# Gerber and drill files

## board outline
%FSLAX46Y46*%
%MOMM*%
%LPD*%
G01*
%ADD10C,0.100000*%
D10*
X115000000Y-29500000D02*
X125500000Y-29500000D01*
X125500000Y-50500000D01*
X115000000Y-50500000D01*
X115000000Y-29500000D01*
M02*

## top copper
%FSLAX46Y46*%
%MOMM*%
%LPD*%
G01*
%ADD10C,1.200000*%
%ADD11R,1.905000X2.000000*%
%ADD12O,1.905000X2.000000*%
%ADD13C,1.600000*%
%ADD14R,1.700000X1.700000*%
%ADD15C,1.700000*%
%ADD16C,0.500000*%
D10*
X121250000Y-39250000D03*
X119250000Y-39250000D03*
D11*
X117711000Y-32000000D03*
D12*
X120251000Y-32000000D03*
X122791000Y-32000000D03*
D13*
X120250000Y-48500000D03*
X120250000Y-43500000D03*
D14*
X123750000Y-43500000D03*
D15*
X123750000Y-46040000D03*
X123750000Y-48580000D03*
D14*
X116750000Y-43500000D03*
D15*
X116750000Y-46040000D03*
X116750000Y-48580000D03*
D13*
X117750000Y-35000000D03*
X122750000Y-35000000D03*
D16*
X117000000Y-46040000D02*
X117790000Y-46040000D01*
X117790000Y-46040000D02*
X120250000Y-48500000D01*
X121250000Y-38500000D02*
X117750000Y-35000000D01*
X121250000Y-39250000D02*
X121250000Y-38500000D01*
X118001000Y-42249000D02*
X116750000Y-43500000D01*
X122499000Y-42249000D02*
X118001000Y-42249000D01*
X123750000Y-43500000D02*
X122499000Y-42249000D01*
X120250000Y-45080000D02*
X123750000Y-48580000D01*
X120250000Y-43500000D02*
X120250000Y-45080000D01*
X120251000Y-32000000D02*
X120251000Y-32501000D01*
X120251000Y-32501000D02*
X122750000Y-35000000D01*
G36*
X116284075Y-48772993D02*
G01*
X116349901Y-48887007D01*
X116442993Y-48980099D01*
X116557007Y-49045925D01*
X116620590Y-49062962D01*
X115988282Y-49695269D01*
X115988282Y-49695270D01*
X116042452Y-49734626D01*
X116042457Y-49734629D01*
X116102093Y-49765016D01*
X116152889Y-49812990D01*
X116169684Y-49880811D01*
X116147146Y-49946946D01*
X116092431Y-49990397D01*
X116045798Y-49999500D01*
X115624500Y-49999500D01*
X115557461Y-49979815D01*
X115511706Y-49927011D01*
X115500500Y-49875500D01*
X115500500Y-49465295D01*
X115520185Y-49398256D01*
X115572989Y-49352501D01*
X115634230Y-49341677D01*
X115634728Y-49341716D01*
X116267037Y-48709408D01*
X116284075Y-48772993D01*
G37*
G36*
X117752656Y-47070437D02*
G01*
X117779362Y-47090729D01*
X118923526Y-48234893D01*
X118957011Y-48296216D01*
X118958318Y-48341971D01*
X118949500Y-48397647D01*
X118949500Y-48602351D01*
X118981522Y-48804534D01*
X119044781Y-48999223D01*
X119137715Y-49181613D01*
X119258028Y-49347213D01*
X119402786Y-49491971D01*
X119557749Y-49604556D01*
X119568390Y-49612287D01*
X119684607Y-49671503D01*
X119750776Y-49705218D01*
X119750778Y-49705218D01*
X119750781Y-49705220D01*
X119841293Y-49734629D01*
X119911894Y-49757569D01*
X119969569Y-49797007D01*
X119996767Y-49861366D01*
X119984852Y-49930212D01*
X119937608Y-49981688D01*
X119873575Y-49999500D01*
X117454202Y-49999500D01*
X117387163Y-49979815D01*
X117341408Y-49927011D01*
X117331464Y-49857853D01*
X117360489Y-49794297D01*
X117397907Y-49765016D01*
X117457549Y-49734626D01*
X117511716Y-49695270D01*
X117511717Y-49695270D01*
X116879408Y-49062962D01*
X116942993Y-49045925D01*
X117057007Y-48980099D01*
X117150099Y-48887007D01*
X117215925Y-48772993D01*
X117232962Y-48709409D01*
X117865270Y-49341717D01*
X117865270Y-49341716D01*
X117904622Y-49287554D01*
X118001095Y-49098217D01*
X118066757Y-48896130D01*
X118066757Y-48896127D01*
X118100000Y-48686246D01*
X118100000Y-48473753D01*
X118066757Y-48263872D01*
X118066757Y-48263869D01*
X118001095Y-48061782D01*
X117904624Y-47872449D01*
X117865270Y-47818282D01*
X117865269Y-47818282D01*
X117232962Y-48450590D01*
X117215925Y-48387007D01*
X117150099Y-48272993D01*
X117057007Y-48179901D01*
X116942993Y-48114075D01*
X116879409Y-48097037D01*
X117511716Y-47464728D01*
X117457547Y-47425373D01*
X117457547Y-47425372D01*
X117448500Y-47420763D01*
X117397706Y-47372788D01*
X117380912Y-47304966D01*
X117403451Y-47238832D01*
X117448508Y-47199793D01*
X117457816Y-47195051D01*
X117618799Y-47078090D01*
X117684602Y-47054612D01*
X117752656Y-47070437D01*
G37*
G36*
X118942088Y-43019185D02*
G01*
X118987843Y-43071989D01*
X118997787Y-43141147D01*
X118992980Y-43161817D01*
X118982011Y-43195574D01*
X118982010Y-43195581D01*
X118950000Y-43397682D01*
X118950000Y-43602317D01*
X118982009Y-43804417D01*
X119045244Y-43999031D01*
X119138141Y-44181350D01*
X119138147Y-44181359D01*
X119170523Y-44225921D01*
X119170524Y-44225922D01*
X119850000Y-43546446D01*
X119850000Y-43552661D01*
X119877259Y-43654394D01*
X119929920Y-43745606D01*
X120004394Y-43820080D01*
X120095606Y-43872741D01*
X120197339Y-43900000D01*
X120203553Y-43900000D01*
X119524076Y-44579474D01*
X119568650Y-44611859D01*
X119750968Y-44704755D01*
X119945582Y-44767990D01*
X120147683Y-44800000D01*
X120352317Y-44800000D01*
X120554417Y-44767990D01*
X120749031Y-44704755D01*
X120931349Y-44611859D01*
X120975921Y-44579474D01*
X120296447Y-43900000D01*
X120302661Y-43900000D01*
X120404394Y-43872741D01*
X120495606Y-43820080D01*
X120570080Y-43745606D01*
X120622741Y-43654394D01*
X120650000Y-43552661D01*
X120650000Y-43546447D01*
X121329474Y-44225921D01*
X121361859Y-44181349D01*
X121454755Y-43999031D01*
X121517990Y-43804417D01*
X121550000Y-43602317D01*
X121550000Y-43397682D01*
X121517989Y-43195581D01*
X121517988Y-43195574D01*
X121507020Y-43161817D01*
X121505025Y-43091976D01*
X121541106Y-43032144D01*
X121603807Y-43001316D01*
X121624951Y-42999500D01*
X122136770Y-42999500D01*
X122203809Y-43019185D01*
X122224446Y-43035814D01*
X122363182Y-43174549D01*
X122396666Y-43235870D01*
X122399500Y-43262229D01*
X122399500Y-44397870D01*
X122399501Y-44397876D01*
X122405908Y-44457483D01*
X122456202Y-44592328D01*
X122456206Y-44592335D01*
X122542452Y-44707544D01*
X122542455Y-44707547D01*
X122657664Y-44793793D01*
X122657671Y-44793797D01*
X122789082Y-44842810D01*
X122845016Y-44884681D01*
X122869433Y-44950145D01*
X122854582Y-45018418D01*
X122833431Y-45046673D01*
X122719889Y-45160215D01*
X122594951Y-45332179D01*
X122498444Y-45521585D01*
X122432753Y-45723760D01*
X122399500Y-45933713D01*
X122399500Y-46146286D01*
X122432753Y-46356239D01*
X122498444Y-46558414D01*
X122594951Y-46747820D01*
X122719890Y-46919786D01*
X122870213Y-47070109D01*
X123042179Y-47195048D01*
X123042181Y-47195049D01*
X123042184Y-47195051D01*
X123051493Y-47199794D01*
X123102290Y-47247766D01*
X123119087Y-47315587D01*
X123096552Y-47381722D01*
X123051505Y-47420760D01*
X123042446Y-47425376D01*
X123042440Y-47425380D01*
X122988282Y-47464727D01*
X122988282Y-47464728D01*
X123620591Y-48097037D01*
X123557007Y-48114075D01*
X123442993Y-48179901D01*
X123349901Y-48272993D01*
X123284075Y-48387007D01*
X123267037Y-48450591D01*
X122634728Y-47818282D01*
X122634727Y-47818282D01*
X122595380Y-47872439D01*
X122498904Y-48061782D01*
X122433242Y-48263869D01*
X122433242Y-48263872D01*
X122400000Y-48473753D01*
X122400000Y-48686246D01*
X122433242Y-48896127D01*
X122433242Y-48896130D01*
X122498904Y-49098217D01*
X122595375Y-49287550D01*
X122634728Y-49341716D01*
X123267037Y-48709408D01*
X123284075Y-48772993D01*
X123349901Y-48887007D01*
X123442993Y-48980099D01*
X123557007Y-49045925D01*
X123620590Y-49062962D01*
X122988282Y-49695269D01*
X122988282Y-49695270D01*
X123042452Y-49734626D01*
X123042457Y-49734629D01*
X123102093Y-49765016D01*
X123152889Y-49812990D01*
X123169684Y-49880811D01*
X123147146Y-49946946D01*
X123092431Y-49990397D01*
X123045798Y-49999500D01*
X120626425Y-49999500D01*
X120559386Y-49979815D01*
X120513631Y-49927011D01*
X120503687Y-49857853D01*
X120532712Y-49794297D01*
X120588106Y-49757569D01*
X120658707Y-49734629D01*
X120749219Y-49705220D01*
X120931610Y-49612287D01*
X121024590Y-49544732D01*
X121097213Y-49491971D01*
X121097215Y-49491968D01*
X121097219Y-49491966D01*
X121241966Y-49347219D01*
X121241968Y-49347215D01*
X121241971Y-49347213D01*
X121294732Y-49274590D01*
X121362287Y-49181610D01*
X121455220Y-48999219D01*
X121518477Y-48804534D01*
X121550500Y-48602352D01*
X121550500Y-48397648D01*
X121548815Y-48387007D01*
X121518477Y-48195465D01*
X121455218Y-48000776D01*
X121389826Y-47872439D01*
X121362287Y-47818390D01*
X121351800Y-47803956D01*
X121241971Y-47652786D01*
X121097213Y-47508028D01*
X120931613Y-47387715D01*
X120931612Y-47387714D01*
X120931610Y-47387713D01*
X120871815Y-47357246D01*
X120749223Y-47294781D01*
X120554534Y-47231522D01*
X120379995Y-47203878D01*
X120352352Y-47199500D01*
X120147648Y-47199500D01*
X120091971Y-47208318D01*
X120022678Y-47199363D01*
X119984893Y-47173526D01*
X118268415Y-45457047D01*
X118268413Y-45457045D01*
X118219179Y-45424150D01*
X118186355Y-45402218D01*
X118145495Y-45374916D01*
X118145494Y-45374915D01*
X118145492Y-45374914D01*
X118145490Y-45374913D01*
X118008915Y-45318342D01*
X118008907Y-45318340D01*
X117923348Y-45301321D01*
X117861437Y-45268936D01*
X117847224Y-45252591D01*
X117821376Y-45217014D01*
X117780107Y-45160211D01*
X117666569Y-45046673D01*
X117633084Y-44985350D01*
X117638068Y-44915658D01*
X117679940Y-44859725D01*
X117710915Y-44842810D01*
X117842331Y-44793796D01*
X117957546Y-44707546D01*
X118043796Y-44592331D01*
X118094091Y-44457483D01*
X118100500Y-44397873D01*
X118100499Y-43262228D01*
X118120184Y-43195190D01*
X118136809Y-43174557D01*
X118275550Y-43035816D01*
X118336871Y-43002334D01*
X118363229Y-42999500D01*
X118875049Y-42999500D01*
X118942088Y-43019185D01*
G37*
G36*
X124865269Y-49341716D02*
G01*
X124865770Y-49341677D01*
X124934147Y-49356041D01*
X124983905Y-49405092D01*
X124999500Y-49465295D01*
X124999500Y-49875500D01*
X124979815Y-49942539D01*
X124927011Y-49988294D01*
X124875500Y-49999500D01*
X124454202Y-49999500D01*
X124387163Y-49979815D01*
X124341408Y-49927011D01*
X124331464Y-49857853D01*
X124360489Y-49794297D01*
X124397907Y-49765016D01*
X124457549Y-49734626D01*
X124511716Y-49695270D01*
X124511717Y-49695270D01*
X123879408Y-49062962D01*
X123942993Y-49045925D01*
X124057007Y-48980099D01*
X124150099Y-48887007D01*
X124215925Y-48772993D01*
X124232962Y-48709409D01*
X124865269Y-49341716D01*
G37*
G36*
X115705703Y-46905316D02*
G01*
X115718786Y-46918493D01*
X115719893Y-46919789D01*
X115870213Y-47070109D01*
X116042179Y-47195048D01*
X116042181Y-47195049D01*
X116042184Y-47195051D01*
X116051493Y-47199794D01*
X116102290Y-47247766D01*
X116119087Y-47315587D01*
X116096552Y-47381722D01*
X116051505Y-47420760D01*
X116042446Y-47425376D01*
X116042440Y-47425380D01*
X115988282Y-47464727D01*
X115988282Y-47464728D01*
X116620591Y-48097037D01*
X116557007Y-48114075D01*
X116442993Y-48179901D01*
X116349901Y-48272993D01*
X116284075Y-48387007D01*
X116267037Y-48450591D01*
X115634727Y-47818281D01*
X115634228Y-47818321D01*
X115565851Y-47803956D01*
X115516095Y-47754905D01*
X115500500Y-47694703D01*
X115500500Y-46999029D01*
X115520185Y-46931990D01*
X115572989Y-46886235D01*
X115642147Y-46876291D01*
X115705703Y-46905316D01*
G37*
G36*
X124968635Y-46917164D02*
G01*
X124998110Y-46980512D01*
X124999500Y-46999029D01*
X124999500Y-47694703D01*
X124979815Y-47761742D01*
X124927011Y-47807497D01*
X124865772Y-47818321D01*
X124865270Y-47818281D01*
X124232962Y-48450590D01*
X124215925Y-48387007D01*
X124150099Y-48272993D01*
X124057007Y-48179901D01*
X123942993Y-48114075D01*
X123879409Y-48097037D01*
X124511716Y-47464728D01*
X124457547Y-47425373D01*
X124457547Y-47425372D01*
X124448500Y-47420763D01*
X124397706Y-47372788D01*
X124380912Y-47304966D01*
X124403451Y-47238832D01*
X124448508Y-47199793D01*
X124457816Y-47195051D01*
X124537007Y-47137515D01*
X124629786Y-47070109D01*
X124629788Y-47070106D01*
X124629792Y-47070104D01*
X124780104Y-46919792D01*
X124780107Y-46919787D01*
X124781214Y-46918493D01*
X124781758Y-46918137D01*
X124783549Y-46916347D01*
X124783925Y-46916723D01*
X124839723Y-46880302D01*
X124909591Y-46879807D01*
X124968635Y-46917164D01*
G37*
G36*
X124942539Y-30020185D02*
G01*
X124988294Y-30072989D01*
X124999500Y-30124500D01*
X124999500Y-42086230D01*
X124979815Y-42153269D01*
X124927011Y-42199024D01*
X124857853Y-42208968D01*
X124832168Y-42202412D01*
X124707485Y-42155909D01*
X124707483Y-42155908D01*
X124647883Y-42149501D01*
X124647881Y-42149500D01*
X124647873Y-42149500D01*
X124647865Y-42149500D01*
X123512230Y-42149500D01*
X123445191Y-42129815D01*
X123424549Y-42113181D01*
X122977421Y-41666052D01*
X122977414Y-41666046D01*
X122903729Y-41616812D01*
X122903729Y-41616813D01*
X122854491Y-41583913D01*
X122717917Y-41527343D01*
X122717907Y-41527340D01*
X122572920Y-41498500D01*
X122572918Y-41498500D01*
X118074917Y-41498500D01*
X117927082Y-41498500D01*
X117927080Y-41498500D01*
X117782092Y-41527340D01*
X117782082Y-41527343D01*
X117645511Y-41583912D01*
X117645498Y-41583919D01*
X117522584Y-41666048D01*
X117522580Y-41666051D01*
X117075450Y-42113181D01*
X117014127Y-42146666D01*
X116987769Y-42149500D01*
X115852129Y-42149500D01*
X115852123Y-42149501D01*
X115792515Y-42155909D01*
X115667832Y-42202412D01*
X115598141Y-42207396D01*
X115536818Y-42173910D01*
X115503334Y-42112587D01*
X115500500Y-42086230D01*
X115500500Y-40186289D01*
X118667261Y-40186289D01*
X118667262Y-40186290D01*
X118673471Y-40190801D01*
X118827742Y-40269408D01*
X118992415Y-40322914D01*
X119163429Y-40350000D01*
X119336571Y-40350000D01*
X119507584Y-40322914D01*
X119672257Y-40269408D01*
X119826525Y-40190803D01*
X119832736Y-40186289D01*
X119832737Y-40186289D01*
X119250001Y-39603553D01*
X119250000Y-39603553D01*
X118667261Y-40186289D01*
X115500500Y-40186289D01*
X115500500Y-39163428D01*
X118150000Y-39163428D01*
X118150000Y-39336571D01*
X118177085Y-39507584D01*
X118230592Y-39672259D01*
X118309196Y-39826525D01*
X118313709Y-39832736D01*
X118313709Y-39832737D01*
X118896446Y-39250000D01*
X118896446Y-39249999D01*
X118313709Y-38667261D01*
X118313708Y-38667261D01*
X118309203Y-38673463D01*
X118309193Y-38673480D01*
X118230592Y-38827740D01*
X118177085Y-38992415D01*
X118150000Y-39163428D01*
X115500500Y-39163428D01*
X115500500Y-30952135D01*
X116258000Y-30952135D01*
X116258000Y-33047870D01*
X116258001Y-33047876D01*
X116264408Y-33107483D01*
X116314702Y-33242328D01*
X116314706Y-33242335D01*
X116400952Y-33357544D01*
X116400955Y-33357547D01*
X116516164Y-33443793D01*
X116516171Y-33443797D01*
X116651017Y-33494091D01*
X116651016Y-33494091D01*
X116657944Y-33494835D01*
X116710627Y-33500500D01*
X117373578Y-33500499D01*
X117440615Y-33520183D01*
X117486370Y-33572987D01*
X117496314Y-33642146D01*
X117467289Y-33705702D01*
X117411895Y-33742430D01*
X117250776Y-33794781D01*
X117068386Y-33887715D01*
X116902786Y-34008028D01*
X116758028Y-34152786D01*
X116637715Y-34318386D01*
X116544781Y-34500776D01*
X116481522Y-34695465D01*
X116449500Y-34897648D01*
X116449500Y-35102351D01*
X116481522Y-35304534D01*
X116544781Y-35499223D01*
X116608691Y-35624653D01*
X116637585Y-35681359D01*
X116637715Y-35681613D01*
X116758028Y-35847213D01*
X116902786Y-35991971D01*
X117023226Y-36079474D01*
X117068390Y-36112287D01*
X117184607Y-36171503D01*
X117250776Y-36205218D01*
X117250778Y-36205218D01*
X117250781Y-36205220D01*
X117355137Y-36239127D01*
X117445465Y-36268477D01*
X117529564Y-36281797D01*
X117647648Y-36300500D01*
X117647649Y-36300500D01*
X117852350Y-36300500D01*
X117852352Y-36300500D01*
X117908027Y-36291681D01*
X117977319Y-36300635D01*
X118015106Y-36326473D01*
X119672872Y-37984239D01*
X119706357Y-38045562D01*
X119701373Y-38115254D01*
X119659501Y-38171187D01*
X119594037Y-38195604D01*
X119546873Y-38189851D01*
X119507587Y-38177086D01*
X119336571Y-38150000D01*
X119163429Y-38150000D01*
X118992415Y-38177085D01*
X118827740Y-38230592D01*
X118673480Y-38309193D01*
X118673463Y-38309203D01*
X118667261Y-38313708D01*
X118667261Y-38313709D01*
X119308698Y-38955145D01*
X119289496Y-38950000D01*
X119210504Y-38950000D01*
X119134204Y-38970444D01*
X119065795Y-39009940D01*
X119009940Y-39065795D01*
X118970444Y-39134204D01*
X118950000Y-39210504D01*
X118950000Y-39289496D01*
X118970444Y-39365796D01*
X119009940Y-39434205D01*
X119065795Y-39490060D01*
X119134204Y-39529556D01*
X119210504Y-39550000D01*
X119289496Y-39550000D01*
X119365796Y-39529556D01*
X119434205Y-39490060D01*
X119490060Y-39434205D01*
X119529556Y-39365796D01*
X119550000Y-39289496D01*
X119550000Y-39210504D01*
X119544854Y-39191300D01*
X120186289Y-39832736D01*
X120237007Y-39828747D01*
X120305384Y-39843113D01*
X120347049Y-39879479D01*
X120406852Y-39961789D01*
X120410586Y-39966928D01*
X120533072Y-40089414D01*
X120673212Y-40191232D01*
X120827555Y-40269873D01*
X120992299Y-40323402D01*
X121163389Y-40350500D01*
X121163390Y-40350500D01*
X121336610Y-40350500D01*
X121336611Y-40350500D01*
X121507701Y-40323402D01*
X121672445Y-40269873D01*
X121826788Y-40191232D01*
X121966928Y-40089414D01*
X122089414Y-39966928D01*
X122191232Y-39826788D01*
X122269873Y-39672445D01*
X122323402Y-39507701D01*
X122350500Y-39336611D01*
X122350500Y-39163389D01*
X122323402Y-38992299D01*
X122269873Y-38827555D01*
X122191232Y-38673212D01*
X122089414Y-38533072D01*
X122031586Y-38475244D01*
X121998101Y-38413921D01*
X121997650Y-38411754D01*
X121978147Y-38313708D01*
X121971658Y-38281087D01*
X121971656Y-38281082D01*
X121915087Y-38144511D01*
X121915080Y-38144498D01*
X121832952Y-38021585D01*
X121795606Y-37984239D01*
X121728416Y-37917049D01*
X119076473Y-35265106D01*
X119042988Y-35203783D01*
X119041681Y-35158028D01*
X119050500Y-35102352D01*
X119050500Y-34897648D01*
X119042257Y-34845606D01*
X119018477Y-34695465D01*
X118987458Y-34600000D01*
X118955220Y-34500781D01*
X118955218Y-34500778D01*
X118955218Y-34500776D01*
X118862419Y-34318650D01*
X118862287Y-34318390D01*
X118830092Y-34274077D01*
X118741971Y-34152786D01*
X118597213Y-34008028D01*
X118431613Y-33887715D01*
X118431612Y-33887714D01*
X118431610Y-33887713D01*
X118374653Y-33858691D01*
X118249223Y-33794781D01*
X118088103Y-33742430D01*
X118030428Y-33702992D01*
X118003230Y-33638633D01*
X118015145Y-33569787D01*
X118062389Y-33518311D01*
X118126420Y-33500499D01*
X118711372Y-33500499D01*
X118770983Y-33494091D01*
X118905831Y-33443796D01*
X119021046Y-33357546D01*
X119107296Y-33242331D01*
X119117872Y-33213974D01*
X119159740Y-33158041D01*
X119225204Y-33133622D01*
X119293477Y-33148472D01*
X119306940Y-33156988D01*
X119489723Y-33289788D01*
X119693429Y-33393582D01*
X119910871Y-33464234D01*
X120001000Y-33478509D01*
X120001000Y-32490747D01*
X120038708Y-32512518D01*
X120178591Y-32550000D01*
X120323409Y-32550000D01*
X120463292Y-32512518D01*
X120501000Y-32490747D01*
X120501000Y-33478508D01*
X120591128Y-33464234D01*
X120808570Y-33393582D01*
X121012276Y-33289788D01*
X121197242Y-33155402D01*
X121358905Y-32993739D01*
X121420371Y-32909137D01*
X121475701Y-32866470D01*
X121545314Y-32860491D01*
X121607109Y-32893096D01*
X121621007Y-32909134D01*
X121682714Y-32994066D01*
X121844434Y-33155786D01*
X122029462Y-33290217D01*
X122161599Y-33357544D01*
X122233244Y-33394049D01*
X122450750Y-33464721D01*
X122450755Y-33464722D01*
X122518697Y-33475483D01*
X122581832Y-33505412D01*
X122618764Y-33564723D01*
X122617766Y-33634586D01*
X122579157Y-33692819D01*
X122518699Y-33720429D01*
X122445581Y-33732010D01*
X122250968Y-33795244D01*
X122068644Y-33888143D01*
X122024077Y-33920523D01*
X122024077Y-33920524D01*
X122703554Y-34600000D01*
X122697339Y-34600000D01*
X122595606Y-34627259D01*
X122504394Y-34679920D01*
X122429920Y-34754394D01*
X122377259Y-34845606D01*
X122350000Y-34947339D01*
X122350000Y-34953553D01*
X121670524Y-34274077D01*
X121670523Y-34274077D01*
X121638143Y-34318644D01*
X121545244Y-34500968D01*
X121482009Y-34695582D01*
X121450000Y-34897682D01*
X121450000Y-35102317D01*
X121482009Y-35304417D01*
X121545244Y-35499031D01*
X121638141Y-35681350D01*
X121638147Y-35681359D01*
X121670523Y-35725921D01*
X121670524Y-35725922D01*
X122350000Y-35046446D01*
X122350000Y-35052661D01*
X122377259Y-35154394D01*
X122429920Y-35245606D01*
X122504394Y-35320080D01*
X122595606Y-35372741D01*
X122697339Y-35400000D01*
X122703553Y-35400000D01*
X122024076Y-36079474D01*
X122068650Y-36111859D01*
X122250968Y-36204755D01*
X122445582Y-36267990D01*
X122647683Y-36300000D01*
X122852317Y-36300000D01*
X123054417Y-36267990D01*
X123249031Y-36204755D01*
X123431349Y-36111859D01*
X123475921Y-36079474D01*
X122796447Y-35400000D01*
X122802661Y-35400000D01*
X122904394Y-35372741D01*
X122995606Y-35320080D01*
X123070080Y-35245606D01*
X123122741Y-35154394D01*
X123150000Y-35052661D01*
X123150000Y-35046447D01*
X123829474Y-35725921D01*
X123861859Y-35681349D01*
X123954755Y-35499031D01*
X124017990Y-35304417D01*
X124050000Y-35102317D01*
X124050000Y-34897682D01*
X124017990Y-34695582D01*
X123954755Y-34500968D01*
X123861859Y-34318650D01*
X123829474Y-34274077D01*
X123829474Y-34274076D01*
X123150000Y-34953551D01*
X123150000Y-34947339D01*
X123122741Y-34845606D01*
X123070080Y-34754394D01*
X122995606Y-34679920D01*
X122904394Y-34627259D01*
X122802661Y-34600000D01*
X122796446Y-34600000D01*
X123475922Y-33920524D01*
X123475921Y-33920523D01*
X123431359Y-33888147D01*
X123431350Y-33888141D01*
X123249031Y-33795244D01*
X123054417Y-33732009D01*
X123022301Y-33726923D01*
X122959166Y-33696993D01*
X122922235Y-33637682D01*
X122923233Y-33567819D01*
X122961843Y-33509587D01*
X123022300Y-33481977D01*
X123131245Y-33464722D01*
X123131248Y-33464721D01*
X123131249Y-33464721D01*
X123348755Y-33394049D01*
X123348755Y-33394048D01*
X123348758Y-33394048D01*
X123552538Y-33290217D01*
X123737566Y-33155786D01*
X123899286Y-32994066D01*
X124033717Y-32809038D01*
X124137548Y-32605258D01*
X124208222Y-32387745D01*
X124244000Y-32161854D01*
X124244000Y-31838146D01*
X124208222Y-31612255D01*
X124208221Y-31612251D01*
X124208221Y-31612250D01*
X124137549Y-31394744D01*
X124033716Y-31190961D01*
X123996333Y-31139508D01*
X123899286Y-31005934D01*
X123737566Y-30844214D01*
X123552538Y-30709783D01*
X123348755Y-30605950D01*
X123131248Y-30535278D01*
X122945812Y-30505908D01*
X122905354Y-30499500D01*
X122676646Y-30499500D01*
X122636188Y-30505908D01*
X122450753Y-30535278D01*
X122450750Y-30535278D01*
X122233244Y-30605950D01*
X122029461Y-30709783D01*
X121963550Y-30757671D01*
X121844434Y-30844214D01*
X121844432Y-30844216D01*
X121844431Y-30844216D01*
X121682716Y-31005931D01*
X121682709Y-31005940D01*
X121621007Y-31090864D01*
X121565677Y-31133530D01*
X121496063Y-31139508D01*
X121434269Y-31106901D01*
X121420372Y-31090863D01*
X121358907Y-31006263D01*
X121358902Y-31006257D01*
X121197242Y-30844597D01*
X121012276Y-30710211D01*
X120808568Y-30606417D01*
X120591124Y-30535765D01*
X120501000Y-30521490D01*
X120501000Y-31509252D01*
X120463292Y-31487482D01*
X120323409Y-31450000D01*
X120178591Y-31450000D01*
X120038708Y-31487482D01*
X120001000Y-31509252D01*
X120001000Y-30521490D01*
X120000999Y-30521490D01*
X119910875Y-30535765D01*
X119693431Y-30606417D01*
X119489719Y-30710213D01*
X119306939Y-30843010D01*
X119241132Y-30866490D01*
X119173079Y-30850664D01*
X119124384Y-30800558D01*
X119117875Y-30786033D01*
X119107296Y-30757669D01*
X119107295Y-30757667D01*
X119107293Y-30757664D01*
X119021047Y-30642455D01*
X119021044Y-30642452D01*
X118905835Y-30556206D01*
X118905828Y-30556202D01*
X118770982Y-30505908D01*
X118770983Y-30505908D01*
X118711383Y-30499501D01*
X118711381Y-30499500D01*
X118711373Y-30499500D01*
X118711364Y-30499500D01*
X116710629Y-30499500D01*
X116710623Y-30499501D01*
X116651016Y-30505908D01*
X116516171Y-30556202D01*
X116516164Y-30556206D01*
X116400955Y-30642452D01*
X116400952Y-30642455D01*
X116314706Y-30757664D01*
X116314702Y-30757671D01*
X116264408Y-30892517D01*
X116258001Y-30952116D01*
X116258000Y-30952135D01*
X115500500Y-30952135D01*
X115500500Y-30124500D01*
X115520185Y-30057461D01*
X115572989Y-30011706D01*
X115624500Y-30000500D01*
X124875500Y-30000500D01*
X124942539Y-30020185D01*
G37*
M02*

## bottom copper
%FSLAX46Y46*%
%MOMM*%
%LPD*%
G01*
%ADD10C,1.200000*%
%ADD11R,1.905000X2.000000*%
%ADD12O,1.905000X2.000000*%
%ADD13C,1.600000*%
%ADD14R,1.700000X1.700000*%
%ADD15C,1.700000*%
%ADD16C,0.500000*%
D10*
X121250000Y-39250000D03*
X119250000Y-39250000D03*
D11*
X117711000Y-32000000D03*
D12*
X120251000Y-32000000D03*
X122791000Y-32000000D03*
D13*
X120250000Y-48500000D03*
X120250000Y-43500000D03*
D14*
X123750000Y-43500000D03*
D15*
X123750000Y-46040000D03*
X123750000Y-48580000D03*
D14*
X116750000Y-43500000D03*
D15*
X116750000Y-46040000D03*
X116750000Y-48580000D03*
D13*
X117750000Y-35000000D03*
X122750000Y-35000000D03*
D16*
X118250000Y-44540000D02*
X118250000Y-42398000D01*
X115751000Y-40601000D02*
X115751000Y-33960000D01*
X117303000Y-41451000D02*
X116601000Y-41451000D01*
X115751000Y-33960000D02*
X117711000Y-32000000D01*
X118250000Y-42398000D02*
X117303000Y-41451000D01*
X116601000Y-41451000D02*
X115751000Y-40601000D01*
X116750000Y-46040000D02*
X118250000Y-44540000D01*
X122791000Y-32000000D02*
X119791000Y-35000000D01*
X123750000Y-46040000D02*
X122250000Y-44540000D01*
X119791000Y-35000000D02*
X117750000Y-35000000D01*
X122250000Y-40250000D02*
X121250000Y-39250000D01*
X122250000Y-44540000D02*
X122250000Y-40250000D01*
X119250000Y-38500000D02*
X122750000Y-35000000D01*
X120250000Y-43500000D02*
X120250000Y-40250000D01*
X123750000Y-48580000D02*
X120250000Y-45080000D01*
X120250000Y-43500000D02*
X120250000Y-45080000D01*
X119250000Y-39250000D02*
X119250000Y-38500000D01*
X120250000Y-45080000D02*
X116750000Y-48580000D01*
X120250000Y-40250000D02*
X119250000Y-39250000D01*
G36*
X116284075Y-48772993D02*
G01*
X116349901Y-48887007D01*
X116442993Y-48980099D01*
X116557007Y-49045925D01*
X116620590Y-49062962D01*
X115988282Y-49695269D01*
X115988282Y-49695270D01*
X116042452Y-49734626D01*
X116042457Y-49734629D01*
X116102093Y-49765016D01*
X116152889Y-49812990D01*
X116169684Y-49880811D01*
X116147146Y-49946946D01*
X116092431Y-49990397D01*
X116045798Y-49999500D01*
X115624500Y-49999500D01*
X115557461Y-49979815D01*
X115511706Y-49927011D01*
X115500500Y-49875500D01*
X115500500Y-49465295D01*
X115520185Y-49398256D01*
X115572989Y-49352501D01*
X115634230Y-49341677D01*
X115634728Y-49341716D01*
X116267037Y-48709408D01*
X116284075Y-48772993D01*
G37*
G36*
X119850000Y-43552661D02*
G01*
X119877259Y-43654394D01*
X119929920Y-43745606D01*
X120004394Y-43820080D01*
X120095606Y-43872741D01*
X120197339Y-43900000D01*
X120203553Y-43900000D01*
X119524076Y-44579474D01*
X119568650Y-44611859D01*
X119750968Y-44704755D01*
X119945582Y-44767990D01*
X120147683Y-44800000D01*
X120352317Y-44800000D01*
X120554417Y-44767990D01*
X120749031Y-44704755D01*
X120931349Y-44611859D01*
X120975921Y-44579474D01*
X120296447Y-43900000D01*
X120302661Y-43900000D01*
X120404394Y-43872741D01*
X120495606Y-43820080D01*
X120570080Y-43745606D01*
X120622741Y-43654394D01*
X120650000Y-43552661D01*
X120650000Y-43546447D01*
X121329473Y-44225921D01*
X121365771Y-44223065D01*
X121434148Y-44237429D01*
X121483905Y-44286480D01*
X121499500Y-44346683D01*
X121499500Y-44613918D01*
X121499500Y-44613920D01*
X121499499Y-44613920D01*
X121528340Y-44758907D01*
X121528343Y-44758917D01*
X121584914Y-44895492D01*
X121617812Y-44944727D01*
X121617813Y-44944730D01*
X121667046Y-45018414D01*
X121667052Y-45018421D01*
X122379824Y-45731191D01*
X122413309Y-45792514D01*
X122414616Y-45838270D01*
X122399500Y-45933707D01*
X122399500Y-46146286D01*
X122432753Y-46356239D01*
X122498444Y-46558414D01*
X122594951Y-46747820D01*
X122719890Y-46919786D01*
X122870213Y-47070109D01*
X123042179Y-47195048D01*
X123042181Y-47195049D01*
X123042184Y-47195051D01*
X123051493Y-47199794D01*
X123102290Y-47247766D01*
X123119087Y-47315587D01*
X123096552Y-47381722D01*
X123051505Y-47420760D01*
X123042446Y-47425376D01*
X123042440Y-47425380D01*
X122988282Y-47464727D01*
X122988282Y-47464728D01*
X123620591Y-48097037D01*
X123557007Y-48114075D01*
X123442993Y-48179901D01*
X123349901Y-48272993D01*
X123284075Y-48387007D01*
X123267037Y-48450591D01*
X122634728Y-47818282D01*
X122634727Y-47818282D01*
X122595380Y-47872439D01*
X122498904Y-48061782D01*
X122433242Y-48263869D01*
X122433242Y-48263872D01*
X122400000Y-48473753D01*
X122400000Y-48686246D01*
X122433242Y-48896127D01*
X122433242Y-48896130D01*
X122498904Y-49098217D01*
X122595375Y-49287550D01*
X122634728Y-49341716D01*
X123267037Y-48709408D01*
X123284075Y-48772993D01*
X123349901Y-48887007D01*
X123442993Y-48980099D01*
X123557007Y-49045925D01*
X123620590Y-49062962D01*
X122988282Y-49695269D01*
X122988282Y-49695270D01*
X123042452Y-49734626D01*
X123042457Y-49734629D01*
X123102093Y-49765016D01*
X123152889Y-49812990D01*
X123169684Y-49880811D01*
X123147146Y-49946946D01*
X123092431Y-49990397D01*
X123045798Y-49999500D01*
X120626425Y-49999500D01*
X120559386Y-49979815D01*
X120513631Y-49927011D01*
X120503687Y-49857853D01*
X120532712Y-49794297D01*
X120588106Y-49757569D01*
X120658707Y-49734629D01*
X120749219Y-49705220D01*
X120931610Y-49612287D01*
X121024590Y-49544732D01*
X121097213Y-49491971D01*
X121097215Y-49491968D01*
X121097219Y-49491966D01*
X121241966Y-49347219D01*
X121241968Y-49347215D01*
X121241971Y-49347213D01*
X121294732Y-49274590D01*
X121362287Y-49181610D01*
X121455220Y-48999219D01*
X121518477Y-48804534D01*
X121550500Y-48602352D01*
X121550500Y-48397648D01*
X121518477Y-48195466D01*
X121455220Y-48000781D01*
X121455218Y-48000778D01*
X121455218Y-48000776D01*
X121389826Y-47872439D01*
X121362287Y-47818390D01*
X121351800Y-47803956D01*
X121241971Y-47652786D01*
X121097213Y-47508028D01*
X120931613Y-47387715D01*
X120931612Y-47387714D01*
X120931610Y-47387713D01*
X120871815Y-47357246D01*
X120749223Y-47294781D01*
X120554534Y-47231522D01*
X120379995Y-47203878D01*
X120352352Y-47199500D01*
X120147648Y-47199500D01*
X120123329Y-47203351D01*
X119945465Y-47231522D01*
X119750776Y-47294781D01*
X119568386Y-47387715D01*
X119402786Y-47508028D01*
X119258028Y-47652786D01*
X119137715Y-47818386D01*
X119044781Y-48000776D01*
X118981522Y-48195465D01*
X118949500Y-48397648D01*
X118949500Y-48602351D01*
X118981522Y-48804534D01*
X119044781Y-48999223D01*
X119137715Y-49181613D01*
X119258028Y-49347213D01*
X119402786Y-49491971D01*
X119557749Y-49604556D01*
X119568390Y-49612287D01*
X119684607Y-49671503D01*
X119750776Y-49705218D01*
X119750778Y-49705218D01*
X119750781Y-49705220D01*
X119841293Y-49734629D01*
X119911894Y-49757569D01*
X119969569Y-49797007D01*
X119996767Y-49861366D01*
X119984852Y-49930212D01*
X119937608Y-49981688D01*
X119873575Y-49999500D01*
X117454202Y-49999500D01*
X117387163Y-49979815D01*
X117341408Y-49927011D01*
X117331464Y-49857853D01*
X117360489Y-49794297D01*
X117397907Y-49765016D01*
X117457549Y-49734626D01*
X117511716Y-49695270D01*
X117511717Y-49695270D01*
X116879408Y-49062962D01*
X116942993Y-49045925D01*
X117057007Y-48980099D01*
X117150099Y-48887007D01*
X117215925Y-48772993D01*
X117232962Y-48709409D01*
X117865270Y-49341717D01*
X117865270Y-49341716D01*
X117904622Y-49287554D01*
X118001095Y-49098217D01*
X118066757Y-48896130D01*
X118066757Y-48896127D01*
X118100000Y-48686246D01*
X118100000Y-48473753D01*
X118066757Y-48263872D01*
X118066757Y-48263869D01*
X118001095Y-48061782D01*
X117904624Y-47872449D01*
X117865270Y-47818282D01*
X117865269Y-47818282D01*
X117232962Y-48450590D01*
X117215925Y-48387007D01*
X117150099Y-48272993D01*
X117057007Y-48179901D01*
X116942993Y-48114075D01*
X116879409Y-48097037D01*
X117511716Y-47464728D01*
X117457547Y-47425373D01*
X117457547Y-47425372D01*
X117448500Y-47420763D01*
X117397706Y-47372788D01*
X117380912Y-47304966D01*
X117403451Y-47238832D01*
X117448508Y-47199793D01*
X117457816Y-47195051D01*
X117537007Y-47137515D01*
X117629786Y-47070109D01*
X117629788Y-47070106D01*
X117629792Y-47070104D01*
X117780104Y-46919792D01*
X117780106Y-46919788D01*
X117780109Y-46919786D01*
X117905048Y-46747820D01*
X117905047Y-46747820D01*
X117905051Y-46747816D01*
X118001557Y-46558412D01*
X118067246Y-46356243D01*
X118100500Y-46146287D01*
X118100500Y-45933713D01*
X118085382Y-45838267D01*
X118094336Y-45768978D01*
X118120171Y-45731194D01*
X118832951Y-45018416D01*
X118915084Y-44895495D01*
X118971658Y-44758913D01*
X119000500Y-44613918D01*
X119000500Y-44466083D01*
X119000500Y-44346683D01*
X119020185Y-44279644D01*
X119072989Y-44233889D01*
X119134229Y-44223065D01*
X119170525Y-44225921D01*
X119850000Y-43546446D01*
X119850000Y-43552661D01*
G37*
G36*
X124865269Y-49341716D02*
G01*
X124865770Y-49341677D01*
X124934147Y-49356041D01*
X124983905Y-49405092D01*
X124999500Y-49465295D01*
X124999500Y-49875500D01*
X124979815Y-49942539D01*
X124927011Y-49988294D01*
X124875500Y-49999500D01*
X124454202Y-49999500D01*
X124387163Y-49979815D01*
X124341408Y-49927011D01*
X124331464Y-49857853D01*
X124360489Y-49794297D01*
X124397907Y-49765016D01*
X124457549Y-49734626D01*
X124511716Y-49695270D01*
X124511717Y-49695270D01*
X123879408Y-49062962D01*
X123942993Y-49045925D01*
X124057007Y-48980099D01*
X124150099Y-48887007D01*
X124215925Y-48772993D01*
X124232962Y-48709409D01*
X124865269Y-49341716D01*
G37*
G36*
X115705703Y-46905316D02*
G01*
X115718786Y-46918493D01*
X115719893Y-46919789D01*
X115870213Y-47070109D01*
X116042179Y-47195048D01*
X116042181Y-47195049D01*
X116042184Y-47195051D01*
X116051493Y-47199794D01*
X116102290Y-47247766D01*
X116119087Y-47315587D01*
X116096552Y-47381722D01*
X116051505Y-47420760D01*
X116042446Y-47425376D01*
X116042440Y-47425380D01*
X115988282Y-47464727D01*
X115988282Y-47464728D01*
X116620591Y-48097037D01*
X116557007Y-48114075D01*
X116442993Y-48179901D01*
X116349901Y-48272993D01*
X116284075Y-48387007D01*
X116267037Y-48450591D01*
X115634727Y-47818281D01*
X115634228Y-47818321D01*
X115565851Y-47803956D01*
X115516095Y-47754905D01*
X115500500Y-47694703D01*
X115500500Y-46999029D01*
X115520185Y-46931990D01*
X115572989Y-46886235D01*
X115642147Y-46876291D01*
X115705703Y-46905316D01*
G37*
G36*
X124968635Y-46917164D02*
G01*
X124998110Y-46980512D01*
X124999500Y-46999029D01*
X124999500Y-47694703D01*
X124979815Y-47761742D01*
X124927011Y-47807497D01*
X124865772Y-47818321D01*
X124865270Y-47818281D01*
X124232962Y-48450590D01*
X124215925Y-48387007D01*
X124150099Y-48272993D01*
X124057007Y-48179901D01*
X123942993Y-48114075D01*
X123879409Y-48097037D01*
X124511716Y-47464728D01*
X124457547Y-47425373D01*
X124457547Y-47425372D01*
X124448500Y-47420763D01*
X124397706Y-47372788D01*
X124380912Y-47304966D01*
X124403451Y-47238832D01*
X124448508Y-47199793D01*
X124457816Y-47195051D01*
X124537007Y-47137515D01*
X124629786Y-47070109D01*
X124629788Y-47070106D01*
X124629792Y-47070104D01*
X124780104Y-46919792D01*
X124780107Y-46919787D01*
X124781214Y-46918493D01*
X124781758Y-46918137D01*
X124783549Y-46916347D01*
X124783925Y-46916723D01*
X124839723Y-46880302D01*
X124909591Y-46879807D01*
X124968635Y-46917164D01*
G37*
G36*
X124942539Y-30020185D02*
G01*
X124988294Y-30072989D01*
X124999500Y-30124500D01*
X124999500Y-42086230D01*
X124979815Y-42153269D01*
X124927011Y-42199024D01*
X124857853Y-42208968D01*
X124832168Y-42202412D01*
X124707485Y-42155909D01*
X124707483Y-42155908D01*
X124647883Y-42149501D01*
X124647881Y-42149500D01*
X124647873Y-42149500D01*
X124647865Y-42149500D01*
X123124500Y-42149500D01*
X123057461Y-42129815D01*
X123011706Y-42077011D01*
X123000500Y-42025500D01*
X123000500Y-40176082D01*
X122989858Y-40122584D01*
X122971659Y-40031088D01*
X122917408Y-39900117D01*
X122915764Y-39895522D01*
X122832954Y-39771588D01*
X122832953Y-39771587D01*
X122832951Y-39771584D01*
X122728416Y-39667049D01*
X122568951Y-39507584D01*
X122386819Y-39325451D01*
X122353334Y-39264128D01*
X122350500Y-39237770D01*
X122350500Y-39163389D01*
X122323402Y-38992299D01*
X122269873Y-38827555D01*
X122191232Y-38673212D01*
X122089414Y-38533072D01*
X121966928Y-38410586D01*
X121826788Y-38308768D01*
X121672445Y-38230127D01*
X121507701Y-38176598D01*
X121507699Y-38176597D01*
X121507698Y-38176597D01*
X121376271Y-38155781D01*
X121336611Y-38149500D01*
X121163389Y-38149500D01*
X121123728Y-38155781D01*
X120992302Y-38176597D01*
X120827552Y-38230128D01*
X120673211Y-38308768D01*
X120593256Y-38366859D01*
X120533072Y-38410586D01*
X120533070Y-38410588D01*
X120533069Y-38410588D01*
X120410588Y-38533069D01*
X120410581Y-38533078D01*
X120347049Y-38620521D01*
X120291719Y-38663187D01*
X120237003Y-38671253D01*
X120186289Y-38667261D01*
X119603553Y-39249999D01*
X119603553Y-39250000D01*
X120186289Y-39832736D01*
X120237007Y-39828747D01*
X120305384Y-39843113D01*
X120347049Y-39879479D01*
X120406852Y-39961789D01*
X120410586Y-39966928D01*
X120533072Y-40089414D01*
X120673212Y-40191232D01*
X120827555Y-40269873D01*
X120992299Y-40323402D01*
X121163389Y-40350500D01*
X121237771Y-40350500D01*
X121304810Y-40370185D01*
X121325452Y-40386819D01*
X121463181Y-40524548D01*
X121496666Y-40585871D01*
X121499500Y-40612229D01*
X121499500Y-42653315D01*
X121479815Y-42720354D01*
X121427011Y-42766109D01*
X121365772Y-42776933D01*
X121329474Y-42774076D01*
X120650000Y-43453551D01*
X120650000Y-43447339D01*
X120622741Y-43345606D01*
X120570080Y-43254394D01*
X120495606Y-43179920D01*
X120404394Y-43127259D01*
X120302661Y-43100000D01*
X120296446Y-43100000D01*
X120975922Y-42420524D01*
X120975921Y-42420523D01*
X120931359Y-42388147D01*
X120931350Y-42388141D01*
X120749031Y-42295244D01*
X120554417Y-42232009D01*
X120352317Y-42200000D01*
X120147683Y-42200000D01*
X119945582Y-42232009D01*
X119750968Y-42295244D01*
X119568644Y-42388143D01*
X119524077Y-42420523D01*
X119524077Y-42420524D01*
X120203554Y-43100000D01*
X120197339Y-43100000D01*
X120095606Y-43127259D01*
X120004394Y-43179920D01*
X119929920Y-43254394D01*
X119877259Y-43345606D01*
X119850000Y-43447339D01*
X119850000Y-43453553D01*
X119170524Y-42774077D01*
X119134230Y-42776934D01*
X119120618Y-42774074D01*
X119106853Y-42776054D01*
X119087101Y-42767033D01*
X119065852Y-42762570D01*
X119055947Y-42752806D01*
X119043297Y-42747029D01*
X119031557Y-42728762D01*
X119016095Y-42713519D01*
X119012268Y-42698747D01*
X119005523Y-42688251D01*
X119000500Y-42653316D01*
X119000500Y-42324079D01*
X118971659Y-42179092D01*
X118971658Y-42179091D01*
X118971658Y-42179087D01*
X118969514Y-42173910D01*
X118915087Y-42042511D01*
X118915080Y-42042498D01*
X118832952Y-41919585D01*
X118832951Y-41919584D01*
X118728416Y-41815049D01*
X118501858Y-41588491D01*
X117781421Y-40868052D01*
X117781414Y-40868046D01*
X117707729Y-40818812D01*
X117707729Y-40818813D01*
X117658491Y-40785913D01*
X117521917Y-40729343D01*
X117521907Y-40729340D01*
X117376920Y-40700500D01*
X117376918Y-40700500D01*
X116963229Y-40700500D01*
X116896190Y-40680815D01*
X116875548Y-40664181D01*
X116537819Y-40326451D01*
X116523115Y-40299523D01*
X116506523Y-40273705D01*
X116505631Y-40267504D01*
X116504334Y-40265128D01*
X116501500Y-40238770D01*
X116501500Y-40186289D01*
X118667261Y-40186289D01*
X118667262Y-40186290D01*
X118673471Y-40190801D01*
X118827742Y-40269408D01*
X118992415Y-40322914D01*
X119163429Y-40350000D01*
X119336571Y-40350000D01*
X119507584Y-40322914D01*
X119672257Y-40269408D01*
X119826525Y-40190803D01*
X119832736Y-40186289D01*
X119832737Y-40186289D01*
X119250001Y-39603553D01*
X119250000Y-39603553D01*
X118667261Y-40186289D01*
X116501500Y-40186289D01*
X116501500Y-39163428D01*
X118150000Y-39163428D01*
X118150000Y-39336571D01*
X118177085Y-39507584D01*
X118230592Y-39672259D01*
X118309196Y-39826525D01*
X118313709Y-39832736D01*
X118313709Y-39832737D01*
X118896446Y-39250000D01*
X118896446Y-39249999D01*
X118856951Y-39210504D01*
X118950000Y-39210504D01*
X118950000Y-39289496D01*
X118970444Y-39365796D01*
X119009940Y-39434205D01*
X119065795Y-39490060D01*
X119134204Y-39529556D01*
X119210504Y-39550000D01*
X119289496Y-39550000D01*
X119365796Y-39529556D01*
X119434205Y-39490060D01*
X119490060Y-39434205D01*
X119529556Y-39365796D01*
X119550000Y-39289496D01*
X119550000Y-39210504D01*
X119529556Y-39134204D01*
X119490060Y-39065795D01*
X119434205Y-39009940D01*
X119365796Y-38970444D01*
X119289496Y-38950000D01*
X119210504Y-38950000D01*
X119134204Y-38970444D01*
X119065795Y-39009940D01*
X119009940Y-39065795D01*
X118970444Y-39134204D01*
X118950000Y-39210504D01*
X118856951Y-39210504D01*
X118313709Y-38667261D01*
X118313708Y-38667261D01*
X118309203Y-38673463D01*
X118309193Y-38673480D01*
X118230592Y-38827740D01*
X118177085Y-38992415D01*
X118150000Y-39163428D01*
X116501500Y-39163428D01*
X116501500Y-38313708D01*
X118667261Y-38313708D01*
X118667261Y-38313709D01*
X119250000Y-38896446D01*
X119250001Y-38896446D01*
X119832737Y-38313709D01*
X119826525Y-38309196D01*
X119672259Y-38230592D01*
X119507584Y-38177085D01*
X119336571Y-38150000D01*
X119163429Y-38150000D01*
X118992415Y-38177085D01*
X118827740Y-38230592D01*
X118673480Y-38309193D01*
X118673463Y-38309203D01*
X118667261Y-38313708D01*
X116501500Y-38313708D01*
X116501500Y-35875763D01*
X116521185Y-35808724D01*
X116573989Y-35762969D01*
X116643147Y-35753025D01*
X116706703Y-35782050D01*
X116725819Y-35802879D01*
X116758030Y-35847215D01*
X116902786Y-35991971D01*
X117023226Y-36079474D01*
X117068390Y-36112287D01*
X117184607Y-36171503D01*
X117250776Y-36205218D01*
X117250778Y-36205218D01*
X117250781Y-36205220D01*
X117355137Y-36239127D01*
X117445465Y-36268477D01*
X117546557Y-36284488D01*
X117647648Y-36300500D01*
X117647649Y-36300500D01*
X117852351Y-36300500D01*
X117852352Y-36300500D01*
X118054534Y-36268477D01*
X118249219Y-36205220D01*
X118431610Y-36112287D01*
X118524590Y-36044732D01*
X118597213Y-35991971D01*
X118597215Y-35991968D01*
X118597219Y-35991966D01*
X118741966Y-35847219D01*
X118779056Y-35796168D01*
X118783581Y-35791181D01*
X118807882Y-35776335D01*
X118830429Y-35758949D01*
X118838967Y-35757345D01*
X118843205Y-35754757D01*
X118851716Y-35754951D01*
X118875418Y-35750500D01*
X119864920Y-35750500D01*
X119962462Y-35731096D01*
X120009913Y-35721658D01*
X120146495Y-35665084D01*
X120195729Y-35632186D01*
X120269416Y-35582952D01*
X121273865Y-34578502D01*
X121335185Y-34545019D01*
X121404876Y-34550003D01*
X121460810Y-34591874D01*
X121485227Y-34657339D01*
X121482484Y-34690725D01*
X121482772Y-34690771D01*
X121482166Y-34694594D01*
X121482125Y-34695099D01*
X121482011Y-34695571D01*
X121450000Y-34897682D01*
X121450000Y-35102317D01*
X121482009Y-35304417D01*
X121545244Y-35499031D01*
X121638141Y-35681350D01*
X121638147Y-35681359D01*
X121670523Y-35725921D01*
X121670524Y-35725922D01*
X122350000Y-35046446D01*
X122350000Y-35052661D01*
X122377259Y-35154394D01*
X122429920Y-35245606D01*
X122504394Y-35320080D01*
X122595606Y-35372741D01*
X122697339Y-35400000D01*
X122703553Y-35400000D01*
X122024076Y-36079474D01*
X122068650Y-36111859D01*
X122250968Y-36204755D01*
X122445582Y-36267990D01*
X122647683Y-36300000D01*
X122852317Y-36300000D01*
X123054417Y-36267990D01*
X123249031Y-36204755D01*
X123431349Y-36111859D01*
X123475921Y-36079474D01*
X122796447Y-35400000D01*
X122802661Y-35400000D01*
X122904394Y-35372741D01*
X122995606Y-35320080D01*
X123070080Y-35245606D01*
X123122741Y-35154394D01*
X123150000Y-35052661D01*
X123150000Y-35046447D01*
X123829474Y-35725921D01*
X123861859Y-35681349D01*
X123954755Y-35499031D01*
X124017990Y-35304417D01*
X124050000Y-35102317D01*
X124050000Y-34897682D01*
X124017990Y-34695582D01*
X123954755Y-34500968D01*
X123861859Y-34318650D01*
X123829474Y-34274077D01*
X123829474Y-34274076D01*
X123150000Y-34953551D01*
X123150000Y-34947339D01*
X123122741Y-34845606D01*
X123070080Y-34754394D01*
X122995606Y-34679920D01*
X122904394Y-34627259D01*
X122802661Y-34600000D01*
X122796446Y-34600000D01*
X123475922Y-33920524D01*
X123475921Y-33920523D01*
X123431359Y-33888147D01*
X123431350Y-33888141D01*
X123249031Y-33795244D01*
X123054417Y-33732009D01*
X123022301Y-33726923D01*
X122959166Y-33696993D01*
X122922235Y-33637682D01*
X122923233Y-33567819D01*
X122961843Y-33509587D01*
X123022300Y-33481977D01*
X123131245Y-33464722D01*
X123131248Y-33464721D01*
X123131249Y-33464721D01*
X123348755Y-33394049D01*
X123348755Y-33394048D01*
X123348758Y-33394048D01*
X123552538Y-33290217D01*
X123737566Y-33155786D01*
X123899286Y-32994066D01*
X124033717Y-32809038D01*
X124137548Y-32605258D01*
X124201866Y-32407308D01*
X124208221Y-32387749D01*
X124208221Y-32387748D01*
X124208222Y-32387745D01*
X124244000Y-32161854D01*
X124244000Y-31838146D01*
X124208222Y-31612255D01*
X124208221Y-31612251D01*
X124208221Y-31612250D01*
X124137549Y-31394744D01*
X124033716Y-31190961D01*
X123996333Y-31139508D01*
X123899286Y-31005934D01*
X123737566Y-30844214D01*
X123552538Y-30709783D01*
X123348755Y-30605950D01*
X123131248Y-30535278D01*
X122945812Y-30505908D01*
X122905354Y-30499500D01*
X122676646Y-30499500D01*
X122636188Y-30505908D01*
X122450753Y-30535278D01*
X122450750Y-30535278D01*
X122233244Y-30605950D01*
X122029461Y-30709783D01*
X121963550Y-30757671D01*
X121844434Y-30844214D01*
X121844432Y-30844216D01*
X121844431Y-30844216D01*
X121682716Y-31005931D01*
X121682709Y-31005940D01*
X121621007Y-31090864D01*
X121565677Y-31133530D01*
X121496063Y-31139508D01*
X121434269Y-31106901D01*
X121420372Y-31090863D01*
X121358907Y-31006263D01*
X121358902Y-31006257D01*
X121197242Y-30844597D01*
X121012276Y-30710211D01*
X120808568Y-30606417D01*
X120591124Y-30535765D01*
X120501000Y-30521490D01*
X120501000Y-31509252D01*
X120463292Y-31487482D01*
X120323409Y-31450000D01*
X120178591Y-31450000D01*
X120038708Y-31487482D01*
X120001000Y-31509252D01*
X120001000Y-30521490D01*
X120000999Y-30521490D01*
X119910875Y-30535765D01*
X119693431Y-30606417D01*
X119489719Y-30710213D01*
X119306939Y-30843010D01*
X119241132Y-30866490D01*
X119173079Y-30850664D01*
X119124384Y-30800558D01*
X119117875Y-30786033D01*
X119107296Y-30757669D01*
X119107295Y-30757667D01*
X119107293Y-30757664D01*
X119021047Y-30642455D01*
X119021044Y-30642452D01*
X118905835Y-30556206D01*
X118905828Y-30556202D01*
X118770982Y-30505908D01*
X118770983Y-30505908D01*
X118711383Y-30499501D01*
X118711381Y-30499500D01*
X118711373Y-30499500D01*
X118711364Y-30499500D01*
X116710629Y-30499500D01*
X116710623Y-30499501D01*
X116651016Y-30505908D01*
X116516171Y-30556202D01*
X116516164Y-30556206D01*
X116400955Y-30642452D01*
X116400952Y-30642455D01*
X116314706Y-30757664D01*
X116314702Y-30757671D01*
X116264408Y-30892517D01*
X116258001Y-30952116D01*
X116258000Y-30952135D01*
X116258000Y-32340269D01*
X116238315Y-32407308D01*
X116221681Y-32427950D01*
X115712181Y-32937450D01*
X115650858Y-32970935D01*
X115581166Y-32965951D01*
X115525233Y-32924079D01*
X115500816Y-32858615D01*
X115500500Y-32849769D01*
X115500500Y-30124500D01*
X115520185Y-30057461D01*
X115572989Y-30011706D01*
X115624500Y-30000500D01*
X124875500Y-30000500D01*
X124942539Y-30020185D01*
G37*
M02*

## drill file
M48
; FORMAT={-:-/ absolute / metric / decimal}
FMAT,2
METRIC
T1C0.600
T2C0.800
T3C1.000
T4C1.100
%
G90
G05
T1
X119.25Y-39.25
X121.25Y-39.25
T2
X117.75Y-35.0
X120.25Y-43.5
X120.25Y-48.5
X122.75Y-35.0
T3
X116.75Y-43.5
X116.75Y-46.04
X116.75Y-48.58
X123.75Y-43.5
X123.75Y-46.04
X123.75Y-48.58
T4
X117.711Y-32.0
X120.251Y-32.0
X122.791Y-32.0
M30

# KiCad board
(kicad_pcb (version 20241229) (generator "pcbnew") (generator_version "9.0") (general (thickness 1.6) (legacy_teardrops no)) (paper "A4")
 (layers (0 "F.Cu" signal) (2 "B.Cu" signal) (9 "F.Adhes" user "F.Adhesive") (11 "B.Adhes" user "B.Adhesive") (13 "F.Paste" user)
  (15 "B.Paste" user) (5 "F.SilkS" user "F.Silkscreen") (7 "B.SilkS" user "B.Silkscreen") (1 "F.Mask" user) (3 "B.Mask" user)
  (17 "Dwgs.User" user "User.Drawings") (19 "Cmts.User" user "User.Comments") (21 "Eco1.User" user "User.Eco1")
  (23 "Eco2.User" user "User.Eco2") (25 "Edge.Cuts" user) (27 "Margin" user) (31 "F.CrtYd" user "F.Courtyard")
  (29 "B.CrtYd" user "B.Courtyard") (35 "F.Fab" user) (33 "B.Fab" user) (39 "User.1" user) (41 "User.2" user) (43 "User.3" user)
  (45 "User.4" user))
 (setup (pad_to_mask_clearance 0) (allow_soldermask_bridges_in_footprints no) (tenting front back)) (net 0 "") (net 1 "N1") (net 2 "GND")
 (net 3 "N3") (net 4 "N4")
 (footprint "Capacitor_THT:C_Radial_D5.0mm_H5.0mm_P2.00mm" (layer "F.Cu") (at 121.25 39.25 180)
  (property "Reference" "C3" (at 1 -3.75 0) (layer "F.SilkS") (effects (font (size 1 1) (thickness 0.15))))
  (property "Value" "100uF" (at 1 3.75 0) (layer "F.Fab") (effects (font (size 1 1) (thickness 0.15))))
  (pad "1" thru_hole circle (at 0 0 180) (size 1.2 1.2) (drill 0.6) (layers "*.Cu" "*.Mask") (remove_unused_layers no) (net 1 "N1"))
  (pad "2" thru_hole circle (at 2 0 180) (size 1.2 1.2) (drill 0.6) (layers "*.Cu" "*.Mask") (remove_unused_layers no) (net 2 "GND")))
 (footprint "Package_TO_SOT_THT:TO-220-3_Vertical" (layer "F.Cu") (at 117.711 32)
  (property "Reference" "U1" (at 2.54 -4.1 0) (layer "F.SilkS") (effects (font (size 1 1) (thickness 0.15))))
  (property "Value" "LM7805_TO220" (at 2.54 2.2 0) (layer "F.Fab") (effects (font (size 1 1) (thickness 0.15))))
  (pad "1" thru_hole rect (at 0 0) (size 1.905 2) (drill 1.1) (layers "*.Cu" "*.Mask") (remove_unused_layers no) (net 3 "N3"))
  (pad "2" thru_hole oval (at 2.54 0) (size 1.905 2) (drill 1.1) (layers "*.Cu" "*.Mask") (remove_unused_layers no) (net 2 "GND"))
  (pad "3" thru_hole oval (at 5.08 0) (size 1.905 2) (drill 1.1) (layers "*.Cu" "*.Mask") (remove_unused_layers no) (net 1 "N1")))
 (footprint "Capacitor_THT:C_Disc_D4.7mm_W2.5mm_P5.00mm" (layer "F.Cu") (at 120.25 48.5 90)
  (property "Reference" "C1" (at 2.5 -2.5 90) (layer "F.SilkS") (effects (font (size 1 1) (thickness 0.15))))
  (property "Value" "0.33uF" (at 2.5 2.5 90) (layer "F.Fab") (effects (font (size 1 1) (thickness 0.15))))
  (pad "1" thru_hole circle (at 0 0 90) (size 1.6 1.6) (drill 0.8) (layers "*.Cu" "*.Mask") (remove_unused_layers no) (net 3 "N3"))
  (pad "2" thru_hole circle (at 5 0 90) (size 1.6 1.6) (drill 0.8) (layers "*.Cu" "*.Mask") (remove_unused_layers no) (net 2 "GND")))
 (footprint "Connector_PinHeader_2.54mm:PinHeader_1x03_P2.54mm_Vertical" (layer "F.Cu") (at 123.75 43.5)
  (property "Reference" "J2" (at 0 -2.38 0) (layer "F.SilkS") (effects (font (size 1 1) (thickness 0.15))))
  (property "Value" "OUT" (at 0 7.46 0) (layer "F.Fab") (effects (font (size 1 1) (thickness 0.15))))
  (pad "1" thru_hole rect (at 0 0) (size 1.7 1.7) (drill 1) (layers "*.Cu" "*.Mask") (remove_unused_layers no) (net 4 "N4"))
  (pad "2" thru_hole circle (at 0 2.54) (size 1.7 1.7) (drill 1) (layers "*.Cu" "*.Mask") (remove_unused_layers no) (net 1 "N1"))
  (pad "3" thru_hole circle (at 0 5.08) (size 1.7 1.7) (drill 1) (layers "*.Cu" "*.Mask") (remove_unused_layers no) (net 2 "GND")))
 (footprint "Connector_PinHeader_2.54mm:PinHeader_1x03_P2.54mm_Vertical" (layer "F.Cu") (at 116.75 43.5)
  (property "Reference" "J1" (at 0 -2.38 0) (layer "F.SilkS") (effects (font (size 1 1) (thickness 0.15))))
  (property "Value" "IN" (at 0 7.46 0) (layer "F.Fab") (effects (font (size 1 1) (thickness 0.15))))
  (pad "1" thru_hole rect (at 0 0) (size 1.7 1.7) (drill 1) (layers "*.Cu" "*.Mask") (remove_unused_layers no) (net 4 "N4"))
  (pad "2" thru_hole circle (at 0 2.54) (size 1.7 1.7) (drill 1) (layers "*.Cu" "*.Mask") (remove_unused_layers no) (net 3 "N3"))
  (pad "3" thru_hole circle (at 0 5.08) (size 1.7 1.7) (drill 1) (layers "*.Cu" "*.Mask") (remove_unused_layers no) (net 2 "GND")))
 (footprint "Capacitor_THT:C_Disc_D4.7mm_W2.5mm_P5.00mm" (layer "F.Cu") (at 117.75 35)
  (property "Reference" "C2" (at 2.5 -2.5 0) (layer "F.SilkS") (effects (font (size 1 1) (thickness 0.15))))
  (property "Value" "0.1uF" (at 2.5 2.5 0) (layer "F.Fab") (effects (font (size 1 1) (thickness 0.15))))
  (pad "1" thru_hole circle (at 0 0) (size 1.6 1.6) (drill 0.8) (layers "*.Cu" "*.Mask") (remove_unused_layers no) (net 1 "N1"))
  (pad "2" thru_hole circle (at 5 0) (size 1.6 1.6) (drill 0.8) (layers "*.Cu" "*.Mask") (remove_unused_layers no) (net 2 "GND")))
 (gr_rect (start 115 29.5) (end 125.5 50.5) (stroke (width 0.1) (type solid)) (fill no) (layer "Edge.Cuts"))
 (segment (start 117 46.04) (end 117.79 46.04) (width 0.5) (layer "F.Cu") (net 3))
 (segment (start 117.79 46.04) (end 120.25 48.5) (width 0.5) (layer "F.Cu") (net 3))
 (segment (start 118.25 44.54) (end 118.25 42.398) (width 0.5) (layer "B.Cu") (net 3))
 (segment (start 115.751 40.601) (end 115.751 33.96) (width 0.5) (layer "B.Cu") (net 3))
 (segment (start 117.303 41.451) (end 116.601 41.451) (width 0.5) (layer "B.Cu") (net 3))
 (segment (start 115.751 33.96) (end 117.711 32) (width 0.5) (layer "B.Cu") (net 3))
 (segment (start 118.25 42.398) (end 117.303 41.451) (width 0.5) (layer "B.Cu") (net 3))
 (segment (start 116.601 41.451) (end 115.751 40.601) (width 0.5) (layer "B.Cu") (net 3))
 (segment (start 116.75 46.04) (end 118.25 44.54) (width 0.5) (layer "B.Cu") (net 3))
 (segment (start 121.25 38.5) (end 117.75 35) (width 0.5) (layer "F.Cu") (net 1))
 (segment (start 121.25 39.25) (end 121.25 38.5) (width 0.5) (layer "F.Cu") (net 1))
 (segment (start 122.791 32) (end 119.791 35) (width 0.5) (layer "B.Cu") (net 1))
 (segment (start 123.75 46.04) (end 122.25 44.54) (width 0.5) (layer "B.Cu") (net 1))
 (segment (start 119.791 35) (end 117.75 35) (width 0.5) (layer "B.Cu") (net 1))
 (segment (start 122.25 40.25) (end 121.25 39.25) (width 0.5) (layer "B.Cu") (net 1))
 (segment (start 122.25 44.54) (end 122.25 40.25) (width 0.5) (layer "B.Cu") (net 1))
 (segment (start 118.001 42.249) (end 116.75 43.5) (width 0.5) (layer "F.Cu") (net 4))
 (segment (start 122.499 42.249) (end 118.001 42.249) (width 0.5) (layer "F.Cu") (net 4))
 (segment (start 123.75 43.5) (end 122.499 42.249) (width 0.5) (layer "F.Cu") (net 4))
 (segment (start 120.25 45.08) (end 123.75 48.58) (width 0.5) (layer "F.Cu") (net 2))
 (segment (start 120.25 43.5) (end 120.25 45.08) (width 0.5) (layer "F.Cu") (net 2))
 (segment (start 120.251 32) (end 120.251 32.501) (width 0.5) (layer "F.Cu") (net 2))
 (segment (start 120.251 32.501) (end 122.75 35) (width 0.5) (layer "F.Cu") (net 2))
 (segment (start 119.25 38.5) (end 122.75 35) (width 0.5) (layer "B.Cu") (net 2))
 (segment (start 120.25 43.5) (end 120.25 40.25) (width 0.5) (layer "B.Cu") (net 2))
 (segment (start 123.75 48.58) (end 120.25 45.08) (width 0.5) (layer "B.Cu") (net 2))
 (segment (start 120.25 43.5) (end 120.25 45.08) (width 0.5) (layer "B.Cu") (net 2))
 (segment (start 119.25 39.25) (end 119.25 38.5) (width 0.5) (layer "B.Cu") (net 2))
 (segment (start 120.25 45.08) (end 116.75 48.58) (width 0.5) (layer "B.Cu") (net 2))
 (segment (start 120.25 40.25) (end 119.25 39.25) (width 0.5) (layer "B.Cu") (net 2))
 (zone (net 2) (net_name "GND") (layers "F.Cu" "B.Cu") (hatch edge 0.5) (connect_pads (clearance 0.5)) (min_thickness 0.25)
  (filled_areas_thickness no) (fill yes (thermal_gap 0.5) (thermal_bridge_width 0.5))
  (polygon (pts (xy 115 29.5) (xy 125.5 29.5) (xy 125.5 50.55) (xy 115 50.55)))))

